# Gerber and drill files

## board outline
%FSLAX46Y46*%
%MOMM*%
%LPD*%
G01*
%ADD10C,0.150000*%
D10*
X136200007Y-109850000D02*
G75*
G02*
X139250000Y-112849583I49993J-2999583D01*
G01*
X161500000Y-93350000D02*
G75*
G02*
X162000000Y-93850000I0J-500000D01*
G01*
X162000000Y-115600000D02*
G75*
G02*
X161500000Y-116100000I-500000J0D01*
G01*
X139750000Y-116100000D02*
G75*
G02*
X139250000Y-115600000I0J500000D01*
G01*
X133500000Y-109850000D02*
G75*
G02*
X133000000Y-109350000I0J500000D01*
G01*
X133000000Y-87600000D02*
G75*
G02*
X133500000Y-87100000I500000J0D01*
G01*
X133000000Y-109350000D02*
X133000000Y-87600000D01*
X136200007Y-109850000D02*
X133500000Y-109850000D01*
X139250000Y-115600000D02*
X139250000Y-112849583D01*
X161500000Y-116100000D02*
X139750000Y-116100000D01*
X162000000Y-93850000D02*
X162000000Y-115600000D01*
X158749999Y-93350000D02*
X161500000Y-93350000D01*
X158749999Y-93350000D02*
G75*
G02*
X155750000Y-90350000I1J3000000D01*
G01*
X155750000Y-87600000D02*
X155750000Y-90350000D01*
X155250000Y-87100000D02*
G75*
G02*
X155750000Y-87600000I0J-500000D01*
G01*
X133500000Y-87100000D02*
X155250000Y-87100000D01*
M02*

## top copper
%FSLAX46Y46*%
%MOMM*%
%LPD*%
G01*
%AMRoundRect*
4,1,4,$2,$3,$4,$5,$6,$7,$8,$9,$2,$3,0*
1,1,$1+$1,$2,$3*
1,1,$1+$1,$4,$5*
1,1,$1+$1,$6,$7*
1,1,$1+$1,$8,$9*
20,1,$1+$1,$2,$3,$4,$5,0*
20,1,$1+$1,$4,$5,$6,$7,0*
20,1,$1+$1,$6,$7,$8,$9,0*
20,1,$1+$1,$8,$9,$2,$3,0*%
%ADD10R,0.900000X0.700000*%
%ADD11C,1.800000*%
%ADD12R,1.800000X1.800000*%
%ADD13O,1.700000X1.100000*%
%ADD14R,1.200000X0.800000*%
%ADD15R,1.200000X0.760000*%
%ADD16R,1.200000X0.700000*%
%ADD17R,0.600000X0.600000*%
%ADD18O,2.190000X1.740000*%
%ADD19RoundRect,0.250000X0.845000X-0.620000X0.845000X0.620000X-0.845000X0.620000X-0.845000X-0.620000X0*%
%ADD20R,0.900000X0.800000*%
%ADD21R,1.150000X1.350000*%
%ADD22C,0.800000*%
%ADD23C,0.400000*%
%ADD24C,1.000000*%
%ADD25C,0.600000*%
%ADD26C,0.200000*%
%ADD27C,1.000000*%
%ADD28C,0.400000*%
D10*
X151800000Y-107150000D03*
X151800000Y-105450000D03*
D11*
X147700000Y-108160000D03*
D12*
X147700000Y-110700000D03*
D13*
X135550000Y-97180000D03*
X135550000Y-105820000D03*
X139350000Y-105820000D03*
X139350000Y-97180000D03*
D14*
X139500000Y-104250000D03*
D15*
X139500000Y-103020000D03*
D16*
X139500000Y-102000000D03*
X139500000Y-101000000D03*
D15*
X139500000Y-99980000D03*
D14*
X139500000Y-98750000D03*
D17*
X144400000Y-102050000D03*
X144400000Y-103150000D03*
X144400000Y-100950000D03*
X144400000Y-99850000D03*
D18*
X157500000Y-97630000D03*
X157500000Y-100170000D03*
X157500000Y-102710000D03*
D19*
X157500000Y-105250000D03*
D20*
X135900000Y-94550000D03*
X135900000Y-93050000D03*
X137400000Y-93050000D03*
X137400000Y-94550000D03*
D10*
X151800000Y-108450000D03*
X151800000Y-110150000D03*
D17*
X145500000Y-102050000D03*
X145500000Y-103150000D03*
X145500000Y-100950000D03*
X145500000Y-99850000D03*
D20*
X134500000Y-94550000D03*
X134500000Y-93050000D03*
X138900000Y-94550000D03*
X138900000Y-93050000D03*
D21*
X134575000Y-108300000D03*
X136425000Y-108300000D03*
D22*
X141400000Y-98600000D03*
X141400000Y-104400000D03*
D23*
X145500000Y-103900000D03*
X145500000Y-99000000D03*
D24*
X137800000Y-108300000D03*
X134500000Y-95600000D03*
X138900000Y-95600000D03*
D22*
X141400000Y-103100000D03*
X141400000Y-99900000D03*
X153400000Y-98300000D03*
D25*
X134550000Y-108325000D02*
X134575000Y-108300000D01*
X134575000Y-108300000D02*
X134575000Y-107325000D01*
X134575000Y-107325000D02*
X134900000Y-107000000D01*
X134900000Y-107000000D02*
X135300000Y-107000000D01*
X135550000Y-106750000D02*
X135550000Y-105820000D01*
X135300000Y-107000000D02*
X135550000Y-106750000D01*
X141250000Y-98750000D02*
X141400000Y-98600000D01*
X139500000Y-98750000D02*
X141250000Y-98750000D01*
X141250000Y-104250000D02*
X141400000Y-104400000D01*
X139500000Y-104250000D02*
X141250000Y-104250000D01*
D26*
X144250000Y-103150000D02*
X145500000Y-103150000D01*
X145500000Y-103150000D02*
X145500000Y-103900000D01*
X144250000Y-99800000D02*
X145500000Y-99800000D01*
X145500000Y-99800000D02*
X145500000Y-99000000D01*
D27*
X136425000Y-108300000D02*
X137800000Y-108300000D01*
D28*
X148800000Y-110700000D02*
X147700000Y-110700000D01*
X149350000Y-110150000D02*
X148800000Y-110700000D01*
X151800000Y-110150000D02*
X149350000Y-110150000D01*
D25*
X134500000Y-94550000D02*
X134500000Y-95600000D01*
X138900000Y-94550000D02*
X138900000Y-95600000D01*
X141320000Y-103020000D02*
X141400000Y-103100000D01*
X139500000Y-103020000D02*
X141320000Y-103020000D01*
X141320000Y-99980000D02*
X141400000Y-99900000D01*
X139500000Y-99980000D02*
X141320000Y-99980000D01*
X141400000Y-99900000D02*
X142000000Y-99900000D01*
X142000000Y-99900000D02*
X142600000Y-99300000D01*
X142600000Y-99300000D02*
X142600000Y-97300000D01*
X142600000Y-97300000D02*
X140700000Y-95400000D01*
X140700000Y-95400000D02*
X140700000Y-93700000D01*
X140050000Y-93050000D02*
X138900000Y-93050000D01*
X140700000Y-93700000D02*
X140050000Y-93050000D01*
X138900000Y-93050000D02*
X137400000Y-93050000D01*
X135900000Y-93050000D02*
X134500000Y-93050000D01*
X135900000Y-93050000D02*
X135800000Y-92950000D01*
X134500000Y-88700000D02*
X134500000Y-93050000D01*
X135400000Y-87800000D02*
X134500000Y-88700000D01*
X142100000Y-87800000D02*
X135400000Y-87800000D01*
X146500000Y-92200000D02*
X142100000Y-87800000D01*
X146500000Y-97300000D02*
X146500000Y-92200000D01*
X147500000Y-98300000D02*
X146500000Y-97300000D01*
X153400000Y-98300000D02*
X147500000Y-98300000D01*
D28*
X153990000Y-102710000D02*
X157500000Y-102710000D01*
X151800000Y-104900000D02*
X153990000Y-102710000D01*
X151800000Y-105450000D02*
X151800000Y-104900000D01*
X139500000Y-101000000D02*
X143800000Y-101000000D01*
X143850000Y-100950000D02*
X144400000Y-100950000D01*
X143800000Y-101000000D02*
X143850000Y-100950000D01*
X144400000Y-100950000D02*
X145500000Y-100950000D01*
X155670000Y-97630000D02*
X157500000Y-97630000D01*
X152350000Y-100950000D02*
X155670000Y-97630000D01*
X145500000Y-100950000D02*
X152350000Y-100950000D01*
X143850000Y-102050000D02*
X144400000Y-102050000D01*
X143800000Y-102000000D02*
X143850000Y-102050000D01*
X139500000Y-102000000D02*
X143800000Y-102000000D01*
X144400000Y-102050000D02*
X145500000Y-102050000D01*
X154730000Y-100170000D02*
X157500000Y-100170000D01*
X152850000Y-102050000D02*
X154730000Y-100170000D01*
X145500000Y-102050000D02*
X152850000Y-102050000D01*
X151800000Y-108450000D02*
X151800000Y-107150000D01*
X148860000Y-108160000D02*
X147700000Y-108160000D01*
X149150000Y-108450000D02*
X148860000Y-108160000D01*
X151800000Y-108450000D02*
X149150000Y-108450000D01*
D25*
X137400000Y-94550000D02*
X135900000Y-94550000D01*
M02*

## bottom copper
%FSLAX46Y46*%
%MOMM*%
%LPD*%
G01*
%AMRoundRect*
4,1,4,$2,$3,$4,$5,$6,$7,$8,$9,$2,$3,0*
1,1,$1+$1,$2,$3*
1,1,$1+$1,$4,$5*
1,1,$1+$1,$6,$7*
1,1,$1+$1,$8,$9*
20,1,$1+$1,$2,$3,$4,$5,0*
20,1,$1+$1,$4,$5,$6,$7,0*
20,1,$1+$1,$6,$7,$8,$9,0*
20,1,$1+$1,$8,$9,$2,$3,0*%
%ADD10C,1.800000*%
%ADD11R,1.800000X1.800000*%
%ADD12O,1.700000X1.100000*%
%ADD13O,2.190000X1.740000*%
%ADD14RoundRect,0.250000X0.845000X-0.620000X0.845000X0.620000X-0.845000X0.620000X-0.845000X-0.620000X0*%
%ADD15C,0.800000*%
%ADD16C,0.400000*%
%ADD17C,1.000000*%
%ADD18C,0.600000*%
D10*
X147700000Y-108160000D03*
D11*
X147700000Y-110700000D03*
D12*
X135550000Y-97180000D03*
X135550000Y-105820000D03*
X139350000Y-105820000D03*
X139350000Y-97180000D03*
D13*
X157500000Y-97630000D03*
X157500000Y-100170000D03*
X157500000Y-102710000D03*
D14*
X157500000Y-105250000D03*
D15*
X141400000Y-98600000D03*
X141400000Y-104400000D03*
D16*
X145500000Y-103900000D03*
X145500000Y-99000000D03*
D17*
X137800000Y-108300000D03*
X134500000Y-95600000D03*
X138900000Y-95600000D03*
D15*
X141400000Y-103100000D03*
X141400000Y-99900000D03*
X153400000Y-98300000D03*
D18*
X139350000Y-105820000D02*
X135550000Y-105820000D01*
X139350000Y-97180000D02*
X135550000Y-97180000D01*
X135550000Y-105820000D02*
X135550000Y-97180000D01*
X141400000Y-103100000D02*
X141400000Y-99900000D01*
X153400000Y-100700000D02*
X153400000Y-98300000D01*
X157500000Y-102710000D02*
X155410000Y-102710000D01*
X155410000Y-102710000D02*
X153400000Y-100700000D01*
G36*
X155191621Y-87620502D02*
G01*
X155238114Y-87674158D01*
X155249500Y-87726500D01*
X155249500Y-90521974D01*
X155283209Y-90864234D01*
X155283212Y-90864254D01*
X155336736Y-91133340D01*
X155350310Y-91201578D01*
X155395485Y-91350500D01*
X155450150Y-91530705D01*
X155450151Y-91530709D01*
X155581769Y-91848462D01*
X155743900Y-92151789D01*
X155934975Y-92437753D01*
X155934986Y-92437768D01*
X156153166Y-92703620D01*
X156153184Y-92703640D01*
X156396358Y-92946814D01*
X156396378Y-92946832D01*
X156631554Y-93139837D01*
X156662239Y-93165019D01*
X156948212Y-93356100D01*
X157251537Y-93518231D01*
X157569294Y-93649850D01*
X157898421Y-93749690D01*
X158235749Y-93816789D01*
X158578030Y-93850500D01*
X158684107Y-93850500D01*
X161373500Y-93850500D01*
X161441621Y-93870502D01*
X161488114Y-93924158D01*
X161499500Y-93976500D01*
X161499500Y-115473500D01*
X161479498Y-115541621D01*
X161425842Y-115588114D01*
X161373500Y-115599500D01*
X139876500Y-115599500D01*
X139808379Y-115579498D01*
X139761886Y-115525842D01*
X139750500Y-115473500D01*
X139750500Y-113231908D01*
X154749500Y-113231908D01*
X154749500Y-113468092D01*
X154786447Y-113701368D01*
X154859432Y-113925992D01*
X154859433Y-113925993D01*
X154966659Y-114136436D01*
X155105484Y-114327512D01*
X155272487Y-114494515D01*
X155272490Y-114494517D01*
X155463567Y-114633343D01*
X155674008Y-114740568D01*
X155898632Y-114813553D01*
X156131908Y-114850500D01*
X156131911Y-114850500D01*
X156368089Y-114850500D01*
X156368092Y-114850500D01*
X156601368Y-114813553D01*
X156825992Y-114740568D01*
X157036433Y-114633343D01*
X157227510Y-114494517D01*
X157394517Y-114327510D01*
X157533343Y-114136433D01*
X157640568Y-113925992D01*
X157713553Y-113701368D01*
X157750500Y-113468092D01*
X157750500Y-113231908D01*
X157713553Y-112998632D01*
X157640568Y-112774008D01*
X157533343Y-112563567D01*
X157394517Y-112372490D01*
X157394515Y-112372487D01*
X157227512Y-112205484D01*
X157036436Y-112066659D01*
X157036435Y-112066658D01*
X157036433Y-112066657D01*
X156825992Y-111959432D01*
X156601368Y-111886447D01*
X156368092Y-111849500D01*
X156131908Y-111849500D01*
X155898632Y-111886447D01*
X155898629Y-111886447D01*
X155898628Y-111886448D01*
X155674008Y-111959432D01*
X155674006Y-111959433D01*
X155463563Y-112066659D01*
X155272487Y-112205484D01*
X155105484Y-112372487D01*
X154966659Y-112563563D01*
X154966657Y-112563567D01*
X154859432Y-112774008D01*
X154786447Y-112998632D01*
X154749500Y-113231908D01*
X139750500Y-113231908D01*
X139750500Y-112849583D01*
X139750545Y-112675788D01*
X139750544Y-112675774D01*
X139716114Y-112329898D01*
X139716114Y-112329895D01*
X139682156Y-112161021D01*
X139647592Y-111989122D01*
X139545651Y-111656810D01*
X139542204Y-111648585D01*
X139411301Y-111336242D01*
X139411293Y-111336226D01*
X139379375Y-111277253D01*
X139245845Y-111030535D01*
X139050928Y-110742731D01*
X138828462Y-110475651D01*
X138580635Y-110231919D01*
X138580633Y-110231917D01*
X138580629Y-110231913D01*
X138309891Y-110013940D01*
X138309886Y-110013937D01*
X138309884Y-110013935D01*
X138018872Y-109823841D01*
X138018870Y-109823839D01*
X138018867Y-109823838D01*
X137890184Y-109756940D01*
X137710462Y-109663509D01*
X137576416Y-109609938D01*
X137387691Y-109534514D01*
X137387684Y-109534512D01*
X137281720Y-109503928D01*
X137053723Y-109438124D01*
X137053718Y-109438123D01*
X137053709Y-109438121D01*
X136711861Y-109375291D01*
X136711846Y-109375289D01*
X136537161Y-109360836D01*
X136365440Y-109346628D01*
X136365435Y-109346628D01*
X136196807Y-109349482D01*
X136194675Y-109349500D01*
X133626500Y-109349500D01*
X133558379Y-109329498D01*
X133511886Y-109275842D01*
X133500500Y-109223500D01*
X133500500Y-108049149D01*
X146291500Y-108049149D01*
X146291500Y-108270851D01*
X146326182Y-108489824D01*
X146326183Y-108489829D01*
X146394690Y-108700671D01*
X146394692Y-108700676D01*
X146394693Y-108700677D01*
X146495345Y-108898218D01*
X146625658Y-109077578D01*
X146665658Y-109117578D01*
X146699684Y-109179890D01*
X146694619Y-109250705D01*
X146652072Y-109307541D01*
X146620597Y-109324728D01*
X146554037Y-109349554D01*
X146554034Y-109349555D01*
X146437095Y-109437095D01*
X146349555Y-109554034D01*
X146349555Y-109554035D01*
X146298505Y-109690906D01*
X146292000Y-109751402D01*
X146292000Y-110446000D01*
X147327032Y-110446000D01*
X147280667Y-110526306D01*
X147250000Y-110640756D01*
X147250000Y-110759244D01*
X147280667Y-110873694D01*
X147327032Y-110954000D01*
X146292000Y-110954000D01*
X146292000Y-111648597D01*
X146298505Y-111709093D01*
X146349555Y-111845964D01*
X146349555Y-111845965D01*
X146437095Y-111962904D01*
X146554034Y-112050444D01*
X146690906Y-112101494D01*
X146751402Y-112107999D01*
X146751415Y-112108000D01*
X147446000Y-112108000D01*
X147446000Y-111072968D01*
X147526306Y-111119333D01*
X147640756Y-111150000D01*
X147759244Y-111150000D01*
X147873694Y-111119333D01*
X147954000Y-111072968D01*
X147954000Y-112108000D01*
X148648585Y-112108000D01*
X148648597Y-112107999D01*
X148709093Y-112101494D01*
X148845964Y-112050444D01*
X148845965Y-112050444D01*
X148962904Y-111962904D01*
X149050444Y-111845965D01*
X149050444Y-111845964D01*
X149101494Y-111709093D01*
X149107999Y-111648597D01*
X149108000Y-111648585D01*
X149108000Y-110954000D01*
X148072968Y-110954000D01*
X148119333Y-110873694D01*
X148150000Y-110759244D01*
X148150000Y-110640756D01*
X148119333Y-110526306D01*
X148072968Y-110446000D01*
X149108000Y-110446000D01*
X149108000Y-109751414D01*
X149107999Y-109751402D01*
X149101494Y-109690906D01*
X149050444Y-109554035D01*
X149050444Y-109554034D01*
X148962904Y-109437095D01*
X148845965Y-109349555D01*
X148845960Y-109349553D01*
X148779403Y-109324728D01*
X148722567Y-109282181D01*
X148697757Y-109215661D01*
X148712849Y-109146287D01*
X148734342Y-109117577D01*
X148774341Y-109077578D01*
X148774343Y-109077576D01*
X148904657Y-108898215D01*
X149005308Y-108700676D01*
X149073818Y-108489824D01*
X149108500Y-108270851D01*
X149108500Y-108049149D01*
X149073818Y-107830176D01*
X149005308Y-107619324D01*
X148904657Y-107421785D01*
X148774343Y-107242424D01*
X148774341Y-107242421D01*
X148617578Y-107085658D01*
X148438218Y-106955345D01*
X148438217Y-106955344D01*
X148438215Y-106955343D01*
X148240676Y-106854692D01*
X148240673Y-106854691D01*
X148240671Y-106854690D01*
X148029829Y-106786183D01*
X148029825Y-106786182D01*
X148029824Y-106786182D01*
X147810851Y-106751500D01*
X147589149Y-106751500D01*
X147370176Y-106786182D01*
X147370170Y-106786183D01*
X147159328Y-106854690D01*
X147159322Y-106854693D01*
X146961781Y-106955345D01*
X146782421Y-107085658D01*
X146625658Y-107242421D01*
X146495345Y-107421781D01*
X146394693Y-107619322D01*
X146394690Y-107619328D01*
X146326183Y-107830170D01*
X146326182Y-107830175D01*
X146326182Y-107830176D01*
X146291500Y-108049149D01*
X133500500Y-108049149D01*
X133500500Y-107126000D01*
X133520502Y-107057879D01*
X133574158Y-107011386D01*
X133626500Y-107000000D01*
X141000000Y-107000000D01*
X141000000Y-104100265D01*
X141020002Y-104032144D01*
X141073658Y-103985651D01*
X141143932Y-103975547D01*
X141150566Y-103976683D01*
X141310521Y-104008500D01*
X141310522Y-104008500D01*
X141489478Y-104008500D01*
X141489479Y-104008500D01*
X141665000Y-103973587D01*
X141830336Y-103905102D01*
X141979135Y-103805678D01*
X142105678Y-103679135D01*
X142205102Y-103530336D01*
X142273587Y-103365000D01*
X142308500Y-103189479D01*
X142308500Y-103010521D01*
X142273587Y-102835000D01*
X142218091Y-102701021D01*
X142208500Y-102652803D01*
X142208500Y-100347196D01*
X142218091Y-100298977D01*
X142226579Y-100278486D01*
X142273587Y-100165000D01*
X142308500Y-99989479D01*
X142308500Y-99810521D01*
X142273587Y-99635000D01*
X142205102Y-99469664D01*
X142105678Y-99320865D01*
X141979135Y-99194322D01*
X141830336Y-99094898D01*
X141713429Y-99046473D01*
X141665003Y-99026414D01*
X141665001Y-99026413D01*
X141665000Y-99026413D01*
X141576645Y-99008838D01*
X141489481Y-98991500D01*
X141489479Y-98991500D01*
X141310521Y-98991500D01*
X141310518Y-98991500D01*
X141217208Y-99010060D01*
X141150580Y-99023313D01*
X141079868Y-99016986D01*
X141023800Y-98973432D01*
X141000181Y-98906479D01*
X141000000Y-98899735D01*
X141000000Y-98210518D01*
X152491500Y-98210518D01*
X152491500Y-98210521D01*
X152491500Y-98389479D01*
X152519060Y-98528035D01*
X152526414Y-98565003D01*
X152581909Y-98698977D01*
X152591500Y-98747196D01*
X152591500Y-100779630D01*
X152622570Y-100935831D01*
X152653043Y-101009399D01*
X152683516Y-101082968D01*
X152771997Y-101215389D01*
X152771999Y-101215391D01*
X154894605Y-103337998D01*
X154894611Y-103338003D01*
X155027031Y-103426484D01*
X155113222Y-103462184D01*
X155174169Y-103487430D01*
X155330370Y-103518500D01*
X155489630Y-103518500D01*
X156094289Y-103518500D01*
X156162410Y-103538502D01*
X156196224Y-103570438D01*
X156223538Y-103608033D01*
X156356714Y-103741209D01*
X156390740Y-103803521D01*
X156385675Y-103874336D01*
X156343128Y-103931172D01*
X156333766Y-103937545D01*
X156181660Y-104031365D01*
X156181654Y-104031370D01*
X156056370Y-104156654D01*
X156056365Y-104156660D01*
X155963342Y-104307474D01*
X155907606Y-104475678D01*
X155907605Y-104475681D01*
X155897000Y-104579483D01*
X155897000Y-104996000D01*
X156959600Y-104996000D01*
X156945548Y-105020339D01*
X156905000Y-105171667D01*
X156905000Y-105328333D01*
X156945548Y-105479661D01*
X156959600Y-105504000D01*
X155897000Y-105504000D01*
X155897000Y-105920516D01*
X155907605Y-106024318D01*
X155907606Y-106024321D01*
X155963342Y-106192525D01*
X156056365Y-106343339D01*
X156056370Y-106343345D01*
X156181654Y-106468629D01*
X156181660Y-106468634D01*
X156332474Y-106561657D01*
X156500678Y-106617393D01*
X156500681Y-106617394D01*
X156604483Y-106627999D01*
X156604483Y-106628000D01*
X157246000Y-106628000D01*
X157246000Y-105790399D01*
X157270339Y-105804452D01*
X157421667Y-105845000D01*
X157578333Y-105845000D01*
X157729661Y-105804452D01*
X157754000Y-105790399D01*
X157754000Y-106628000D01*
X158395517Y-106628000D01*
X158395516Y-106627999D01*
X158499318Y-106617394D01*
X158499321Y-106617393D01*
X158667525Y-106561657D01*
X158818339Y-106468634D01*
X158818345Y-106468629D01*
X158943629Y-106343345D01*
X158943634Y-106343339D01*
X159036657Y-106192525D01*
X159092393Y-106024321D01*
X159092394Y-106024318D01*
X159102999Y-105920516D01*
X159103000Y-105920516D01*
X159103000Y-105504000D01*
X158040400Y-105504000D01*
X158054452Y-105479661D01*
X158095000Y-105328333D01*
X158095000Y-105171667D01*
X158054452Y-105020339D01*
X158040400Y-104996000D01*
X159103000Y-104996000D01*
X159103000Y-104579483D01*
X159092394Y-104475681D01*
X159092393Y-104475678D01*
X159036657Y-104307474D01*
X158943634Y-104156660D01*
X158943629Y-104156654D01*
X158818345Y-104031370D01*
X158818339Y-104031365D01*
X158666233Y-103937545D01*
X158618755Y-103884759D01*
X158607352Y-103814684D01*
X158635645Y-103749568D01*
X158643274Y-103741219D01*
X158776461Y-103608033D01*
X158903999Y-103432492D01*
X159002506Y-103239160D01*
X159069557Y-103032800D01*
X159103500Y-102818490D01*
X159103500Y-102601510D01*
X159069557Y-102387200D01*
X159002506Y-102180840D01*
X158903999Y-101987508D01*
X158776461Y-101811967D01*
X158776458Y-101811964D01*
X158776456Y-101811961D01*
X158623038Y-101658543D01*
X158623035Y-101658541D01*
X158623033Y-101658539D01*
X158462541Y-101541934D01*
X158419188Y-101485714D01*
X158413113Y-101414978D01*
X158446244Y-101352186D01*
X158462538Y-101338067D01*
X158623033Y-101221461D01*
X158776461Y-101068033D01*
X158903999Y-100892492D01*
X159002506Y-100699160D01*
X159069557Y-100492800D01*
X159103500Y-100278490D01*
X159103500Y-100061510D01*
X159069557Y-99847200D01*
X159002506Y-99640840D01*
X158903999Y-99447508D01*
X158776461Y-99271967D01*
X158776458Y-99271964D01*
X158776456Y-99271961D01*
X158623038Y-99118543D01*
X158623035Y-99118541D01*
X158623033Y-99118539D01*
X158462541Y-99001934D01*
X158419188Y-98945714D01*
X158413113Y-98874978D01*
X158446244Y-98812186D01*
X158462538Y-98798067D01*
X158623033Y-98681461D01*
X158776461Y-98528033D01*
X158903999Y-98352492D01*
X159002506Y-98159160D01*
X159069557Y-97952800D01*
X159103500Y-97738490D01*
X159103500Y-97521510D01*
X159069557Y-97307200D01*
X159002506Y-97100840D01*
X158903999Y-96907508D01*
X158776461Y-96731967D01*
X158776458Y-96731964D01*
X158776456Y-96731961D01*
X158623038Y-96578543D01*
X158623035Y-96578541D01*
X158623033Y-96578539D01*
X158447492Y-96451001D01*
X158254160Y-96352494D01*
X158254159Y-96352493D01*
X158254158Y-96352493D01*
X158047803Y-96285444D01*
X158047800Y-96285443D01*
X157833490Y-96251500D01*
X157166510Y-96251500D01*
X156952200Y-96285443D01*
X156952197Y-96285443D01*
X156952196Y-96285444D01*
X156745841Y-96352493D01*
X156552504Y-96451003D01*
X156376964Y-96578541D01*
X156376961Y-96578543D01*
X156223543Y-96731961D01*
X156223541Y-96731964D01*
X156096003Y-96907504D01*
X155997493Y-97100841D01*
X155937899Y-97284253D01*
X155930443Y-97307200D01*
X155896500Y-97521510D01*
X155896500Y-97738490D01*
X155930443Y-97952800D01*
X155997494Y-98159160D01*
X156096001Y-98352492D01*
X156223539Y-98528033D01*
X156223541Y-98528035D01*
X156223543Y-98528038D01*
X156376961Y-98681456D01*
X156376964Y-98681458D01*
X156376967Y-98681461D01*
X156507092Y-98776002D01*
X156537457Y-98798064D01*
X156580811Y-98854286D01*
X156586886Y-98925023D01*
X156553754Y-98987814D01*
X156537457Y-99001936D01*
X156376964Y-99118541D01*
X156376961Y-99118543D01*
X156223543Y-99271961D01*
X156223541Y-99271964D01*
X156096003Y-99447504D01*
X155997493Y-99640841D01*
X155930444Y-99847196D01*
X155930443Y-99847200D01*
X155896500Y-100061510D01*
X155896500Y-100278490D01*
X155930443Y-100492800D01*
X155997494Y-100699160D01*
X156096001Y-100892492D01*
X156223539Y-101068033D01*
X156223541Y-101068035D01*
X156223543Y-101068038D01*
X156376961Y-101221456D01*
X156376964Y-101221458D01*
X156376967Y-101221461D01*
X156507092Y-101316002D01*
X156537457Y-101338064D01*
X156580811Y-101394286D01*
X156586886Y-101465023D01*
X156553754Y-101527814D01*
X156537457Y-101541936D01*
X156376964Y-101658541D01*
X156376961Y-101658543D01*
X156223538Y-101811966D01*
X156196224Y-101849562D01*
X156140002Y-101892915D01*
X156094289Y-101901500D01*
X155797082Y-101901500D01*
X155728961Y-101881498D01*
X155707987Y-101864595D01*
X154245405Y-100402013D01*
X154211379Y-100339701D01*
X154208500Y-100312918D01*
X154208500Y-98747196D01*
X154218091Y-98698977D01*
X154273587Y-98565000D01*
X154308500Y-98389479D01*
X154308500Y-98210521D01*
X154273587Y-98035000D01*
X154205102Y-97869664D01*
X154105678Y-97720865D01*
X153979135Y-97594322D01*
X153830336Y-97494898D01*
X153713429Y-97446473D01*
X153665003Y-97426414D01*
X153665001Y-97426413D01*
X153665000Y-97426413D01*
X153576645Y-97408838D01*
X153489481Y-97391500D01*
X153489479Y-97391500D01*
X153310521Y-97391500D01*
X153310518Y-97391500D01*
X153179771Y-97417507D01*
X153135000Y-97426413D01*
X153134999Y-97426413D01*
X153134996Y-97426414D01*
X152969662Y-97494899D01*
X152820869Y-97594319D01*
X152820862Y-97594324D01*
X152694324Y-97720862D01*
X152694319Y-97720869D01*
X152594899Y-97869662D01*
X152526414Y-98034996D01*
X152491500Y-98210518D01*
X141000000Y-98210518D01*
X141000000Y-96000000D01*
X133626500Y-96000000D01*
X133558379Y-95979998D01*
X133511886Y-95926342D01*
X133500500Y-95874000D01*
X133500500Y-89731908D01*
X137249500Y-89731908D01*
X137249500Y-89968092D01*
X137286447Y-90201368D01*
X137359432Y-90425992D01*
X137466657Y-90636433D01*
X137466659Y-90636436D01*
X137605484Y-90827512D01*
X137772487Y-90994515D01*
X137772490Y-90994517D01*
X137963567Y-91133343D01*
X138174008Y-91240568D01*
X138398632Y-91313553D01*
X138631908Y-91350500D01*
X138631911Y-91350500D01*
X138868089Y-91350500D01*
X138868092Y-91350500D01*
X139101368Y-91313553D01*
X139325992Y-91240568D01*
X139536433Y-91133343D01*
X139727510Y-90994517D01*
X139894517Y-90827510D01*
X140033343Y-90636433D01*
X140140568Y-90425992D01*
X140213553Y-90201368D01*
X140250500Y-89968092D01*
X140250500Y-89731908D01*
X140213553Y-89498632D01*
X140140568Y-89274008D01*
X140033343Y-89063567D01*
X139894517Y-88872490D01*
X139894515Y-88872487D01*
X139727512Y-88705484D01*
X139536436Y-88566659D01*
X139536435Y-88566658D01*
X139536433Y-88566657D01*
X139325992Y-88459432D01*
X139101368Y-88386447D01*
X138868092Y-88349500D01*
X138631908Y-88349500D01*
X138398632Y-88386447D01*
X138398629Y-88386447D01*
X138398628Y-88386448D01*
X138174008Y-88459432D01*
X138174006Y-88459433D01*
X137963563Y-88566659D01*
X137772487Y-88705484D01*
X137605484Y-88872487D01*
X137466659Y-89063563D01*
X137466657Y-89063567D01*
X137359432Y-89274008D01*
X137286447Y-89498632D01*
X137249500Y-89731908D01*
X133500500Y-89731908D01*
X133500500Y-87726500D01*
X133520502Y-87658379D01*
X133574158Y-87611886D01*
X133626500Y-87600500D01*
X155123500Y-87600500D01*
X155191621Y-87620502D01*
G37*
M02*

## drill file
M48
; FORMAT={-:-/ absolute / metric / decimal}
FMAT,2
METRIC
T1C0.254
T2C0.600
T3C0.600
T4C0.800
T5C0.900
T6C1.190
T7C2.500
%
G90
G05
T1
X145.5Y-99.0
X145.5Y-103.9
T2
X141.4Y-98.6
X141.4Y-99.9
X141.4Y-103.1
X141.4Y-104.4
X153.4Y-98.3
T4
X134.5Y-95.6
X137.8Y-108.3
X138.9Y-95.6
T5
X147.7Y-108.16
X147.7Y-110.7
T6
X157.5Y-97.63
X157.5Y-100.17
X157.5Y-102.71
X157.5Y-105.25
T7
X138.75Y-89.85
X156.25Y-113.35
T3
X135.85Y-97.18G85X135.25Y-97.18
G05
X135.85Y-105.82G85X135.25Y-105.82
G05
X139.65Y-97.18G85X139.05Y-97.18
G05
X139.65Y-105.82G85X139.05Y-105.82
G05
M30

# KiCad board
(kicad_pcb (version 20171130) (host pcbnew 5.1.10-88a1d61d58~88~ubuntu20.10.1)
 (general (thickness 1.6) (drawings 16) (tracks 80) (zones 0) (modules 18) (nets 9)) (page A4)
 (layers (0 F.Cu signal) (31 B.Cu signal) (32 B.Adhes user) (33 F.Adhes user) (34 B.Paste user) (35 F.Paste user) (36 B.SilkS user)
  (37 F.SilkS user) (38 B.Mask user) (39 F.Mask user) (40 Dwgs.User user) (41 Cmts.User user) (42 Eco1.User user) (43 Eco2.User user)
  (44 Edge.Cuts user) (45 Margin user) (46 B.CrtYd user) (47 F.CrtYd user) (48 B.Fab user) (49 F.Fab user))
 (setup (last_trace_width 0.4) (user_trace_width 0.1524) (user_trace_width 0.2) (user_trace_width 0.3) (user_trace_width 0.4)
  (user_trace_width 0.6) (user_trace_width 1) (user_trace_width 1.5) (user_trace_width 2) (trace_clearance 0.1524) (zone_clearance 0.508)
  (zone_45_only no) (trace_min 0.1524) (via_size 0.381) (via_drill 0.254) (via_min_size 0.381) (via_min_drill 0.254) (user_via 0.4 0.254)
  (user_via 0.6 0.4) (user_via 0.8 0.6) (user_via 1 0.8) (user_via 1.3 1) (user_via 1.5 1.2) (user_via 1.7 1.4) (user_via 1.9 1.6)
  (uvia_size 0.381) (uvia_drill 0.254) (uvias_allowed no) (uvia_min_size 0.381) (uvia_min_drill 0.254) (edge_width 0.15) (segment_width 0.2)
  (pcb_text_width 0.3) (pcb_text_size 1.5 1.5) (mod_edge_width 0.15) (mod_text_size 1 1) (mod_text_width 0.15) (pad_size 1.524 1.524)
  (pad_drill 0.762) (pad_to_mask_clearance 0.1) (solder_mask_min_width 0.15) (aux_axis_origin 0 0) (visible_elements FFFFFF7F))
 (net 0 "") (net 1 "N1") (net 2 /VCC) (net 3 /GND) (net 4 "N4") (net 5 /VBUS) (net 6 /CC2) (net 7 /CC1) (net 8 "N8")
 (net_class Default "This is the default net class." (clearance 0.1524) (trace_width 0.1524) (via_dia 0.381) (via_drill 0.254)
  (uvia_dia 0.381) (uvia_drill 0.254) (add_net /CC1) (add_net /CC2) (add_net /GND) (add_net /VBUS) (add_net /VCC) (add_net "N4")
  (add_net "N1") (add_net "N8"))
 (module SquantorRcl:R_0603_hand (layer F.Cu) (at 151.8 106.3 270)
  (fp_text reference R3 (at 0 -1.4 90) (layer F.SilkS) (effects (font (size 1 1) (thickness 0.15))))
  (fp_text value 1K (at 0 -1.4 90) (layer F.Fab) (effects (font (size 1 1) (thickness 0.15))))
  (pad 2 smd rect (at 0.85 0 270) (size 0.7 0.9) (layers F.Cu F.Paste F.Mask) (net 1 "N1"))
  (pad 1 smd rect (at -0.85 0 270) (size 0.7 0.9) (layers F.Cu F.Paste F.Mask) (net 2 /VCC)))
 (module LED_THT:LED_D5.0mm (layer F.Cu) (at 147.7 110.7 90)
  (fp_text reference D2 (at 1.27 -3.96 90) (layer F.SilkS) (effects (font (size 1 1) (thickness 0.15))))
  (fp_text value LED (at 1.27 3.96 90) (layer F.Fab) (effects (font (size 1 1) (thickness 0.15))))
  (pad 2 thru_hole circle (at 2.54 0 90) (size 1.8 1.8) (drill 0.9) (layers *.Cu *.Mask) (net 1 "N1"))
  (pad 1 thru_hole rect (at 0 0 90) (size 1.8 1.8) (drill 0.9) (layers *.Cu *.Mask) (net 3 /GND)))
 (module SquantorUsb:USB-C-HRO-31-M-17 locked (layer F.Cu) (at 139.5 101.5 270)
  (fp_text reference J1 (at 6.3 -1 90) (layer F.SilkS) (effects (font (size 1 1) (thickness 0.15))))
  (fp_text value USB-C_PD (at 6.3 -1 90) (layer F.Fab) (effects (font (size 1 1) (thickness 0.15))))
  (pad S thru_hole oval (at -4.32 3.95 270) (size 1.1 1.7) (drill oval 0.6 1.2) (layers *.Cu *.Mask) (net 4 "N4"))
  (pad S thru_hole oval (at 4.32 3.95 270) (size 1.1 1.7) (drill oval 0.6 1.2) (layers *.Cu *.Mask) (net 4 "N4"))
  (pad S thru_hole oval (at 4.32 0.15 270) (size 1.1 1.7) (drill oval 0.6 1.2) (layers *.Cu *.Mask) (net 4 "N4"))
  (pad S thru_hole oval (at -4.32 0.15 270) (size 1.1 1.7) (drill oval 0.6 1.2) (layers *.Cu *.Mask) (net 4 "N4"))
  (pad A12 smd rect (at 2.75 0 270) (size 0.8 1.2) (layers F.Cu F.Paste F.Mask) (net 3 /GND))
  (pad A9 smd rect (at 1.52 0 270) (size 0.76 1.2) (layers F.Cu F.Paste F.Mask) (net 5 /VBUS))
  (pad B5 smd rect (at 0.5 0 270) (size 0.7 1.2) (layers F.Cu F.Paste F.Mask) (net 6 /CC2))
  (pad A5 smd rect (at -0.5 0 270) (size 0.7 1.2) (layers F.Cu F.Paste F.Mask) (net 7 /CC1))
  (pad B9 smd rect (at -1.52 0 270) (size 0.76 1.2) (layers F.Cu F.Paste F.Mask) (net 5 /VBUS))
  (pad B12 smd rect (at -2.75 0 270) (size 0.8 1.2) (layers F.Cu F.Paste F.Mask) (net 3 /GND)))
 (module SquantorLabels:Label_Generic (layer B.Cu) (at 148.5 104.75 180)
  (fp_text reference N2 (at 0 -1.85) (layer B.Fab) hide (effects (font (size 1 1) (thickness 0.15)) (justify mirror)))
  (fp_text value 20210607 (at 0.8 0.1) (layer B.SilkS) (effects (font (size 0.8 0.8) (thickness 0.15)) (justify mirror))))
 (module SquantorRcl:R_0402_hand (layer F.Cu) (at 144.4 102.6 90)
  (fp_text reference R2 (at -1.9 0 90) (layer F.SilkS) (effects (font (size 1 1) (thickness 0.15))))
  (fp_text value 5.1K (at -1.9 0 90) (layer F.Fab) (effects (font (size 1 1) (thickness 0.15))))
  (pad 2 smd rect (at 0.55 0 90) (size 0.6 0.6) (layers F.Cu F.Paste F.Mask) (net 6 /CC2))
  (pad 1 smd rect (at -0.55 0 90) (size 0.6 0.6) (layers F.Cu F.Paste F.Mask) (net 3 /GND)))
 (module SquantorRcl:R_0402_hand (layer F.Cu) (at 144.4 100.4 270)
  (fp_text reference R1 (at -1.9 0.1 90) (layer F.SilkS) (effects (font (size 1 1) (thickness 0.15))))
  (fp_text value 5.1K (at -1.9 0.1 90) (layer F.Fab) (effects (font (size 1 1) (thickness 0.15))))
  (pad 2 smd rect (at 0.55 0 270) (size 0.6 0.6) (layers F.Cu F.Paste F.Mask) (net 7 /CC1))
  (pad 1 smd rect (at -0.55 0 270) (size 0.6 0.6) (layers F.Cu F.Paste F.Mask) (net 3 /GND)))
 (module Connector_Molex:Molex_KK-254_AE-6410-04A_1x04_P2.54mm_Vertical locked (layer F.Cu) (at 157.5 105.25 90)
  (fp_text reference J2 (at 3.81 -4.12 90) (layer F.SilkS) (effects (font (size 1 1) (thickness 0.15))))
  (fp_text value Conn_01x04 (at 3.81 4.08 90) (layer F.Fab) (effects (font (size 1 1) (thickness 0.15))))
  (pad 4 thru_hole oval (at 7.62 0 90) (size 1.74 2.19) (drill 1.19) (layers *.Cu *.Mask) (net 7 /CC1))
  (pad 3 thru_hole oval (at 5.08 0 90) (size 1.74 2.19) (drill 1.19) (layers *.Cu *.Mask) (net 6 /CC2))
  (pad 2 thru_hole oval (at 2.54 0 90) (size 1.74 2.19) (drill 1.19) (layers *.Cu *.Mask) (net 2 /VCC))
  (pad 1 thru_hole roundrect (at 0 0 90) (size 1.74 2.19) (drill 1.19) (layers *.Cu *.Mask) (roundrect_rratio 0.143678) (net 3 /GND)))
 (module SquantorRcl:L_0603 (layer F.Cu) (at 135.9 93.8 270)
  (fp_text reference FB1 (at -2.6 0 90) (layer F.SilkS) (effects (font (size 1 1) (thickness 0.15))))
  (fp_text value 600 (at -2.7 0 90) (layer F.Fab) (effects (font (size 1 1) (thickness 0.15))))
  (pad 2 smd rect (at 0.75 0 270) (size 0.8 0.9) (layers F.Cu F.Paste F.Mask) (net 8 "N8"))
  (pad 1 smd rect (at -0.75 0 270) (size 0.8 0.9) (layers F.Cu F.Paste F.Mask) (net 2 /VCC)))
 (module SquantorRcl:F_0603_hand (layer F.Cu) (at 137.4 93.8 90)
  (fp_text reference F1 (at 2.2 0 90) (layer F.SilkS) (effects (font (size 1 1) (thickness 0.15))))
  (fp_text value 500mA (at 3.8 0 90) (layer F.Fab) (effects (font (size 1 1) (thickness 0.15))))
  (pad 2 smd rect (at 0.75 0 90) (size 0.8 0.9) (layers F.Cu F.Paste F.Mask) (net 5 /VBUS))
  (pad 1 smd rect (at -0.75 0 90) (size 0.8 0.9) (layers F.Cu F.Paste F.Mask) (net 8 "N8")))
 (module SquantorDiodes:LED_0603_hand (layer F.Cu) (at 151.8 109.3 90)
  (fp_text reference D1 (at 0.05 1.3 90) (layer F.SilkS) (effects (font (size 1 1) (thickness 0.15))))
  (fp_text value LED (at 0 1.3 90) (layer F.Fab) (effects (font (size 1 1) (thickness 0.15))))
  (pad 2 smd rect (at 0.85 0 90) (size 0.7 0.9) (layers F.Cu F.Paste F.Mask) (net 1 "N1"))
  (pad 1 smd rect (at -0.85 0 90) (size 0.7 0.9) (layers F.Cu F.Paste F.Mask) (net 3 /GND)))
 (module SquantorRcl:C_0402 (layer F.Cu) (at 145.5 102.6 90)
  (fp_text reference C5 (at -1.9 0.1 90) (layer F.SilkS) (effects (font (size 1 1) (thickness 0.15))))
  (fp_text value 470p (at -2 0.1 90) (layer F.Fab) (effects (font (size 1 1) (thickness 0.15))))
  (pad 2 smd rect (at 0.55 0 90) (size 0.6 0.6) (layers F.Cu F.Paste F.Mask) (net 6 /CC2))
  (pad 1 smd rect (at -0.55 0 90) (size 0.6 0.6) (layers F.Cu F.Paste F.Mask) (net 3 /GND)))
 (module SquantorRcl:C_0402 (layer F.Cu) (at 145.5 100.4 270)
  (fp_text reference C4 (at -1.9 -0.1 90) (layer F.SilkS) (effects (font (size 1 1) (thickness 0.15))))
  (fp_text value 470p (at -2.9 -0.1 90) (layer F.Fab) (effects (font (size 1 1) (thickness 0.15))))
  (pad 2 smd rect (at 0.55 0 270) (size 0.6 0.6) (layers F.Cu F.Paste F.Mask) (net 7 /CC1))
  (pad 1 smd rect (at -0.55 0 270) (size 0.6 0.6) (layers F.Cu F.Paste F.Mask) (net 3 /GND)))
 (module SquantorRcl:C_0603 (layer F.Cu) (at 134.5 93.8 270)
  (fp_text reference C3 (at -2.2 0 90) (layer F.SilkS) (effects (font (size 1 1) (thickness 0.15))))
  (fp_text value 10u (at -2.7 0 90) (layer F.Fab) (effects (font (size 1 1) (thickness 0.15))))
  (pad 2 smd rect (at 0.75 0 270) (size 0.8 0.9) (layers F.Cu F.Paste F.Mask) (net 3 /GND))
  (pad 1 smd rect (at -0.75 0 270) (size 0.8 0.9) (layers F.Cu F.Paste F.Mask) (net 2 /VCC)))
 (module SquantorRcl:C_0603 (layer F.Cu) (at 138.9 93.8 270)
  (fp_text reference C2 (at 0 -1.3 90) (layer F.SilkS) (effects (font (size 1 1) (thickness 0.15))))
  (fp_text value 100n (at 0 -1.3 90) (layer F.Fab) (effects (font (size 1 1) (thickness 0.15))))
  (pad 2 smd rect (at 0.75 0 270) (size 0.8 0.9) (layers F.Cu F.Paste F.Mask) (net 3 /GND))
  (pad 1 smd rect (at -0.75 0 270) (size 0.8 0.9) (layers F.Cu F.Paste F.Mask) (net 5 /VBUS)))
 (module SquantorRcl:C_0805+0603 (layer F.Cu) (at 135.5 108.3)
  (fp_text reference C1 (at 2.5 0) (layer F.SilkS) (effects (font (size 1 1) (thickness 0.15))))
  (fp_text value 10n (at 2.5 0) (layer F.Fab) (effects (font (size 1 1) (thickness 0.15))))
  (pad 1 smd rect (at -0.925 0) (size 1.15 1.35) (layers F.Cu F.Paste F.Mask) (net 4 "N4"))
  (pad 2 smd rect (at 0.925 0) (size 1.15 1.35) (layers F.Cu F.Paste F.Mask) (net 3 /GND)))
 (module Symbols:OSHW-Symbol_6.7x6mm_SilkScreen (layer B.Cu) (at 148 101 180)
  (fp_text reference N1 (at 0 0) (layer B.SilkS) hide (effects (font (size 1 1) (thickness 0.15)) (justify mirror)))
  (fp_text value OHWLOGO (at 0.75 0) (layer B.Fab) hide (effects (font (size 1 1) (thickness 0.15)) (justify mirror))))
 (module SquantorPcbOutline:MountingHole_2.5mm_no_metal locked (layer F.Cu) (at 138.75 89.85)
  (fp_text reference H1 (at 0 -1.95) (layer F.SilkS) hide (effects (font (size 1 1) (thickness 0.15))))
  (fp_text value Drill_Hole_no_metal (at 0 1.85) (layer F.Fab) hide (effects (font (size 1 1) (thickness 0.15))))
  (pad "" np_thru_hole circle (at 0 0) (size 2.5 2.5) (drill 2.5) (layers *.Cu *.Mask)))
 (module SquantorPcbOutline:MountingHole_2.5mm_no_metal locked (layer F.Cu) (at 156.25 113.35)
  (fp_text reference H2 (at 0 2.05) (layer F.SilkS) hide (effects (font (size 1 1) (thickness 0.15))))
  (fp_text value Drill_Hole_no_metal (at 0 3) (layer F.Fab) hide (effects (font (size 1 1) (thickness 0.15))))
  (pad "" np_thru_hole circle (at 0 0) (size 2.5 2.5) (drill 2.5) (layers *.Cu *.Mask)))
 (gr_arc (start 136.25 112.849583) (end 139.25 112.849583) (angle -90.95484125) (layer Edge.Cuts) (width 0.15))
 (gr_arc (start 161.5 93.85) (end 162 93.85) (angle -90) (layer Edge.Cuts) (width 0.15))
 (gr_arc (start 161.5 115.6) (end 161.5 116.1) (angle -90) (layer Edge.Cuts) (width 0.15))
 (gr_arc (start 139.75 115.6) (end 139.25 115.6) (angle -90) (layer Edge.Cuts) (width 0.15))
 (gr_arc (start 133.5 109.35) (end 133 109.35) (angle -90) (layer Edge.Cuts) (width 0.15))
 (gr_arc (start 133.5 87.6) (end 133.5 87.1) (angle -90) (layer Edge.Cuts) (width 0.15))
 (gr_line (start 133 109.35) (end 133 87.6) (layer Edge.Cuts) (width 0.15))
 (gr_line (start 136.200007 109.85) (end 133.5 109.85) (layer Edge.Cuts) (width 0.15))
 (gr_line (start 139.25 115.6) (end 139.25 112.849583) (layer Edge.Cuts) (width 0.15))
 (gr_line (start 161.5 116.1) (end 139.75 116.1) (layer Edge.Cuts) (width 0.15))
 (gr_line (start 162 93.85) (end 162 115.6) (layer Edge.Cuts) (width 0.15))
 (gr_line (start 158.749999 93.35) (end 161.5 93.35) (layer Edge.Cuts) (width 0.15))
 (gr_arc (start 158.75 90.35) (end 155.75 90.35) (angle -89.9999809) (layer Edge.Cuts) (width 0.15))
 (gr_line (start 155.75 87.6) (end 155.75 90.35) (layer Edge.Cuts) (width 0.15))
 (gr_arc (start 155.25 87.6) (end 155.75 87.6) (angle -90) (layer Edge.Cuts) (width 0.15))
 (gr_line (start 133.5 87.1) (end 155.25 87.1) (layer Edge.Cuts) (width 0.15))
 (segment (start 139.35 105.82) (end 135.55 105.82) (width 0.6) (layer B.Cu) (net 4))
 (segment (start 139.35 97.18) (end 135.55 97.18) (width 0.6) (layer B.Cu) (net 4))
 (segment (start 135.55 105.82) (end 135.55 97.18) (width 0.6) (layer B.Cu) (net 4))
 (segment (start 134.55 108.325) (end 134.575 108.3) (width 0.6) (layer F.Cu) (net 4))
 (segment (start 134.575 108.3) (end 134.575 107.325) (width 0.6) (layer F.Cu) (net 4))
 (segment (start 134.575 107.325) (end 134.9 107) (width 0.6) (layer F.Cu) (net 4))
 (segment (start 134.9 107) (end 135.3 107) (width 0.6) (layer F.Cu) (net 4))
 (segment (start 135.55 106.75) (end 135.55 105.82) (width 0.6) (layer F.Cu) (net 4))
 (segment (start 135.3 107) (end 135.55 106.75) (width 0.6) (layer F.Cu) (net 4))
 (via (at 141.4 98.6) (size 0.8) (drill 0.6) (layers F.Cu B.Cu) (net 3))
 (segment (start 141.25 98.75) (end 141.4 98.6) (width 0.6) (layer F.Cu) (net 3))
 (segment (start 139.5 98.75) (end 141.25 98.75) (width 0.6) (layer F.Cu) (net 3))
 (via (at 141.4 104.4) (size 0.8) (drill 0.6) (layers F.Cu B.Cu) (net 3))
 (segment (start 141.25 104.25) (end 141.4 104.4) (width 0.6) (layer F.Cu) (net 3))
 (segment (start 139.5 104.25) (end 141.25 104.25) (width 0.6) (layer F.Cu) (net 3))
 (segment (start 144.25 103.15) (end 145.5 103.15) (width 0.2) (layer F.Cu) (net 3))
 (via (at 145.5 103.9) (size 0.4) (drill 0.254) (layers F.Cu B.Cu) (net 3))
 (segment (start 145.5 103.15) (end 145.5 103.9) (width 0.2) (layer F.Cu) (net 3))
 (segment (start 144.25 99.8) (end 145.5 99.8) (width 0.2) (layer F.Cu) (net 3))
 (via (at 145.5 99) (size 0.4) (drill 0.254) (layers F.Cu B.Cu) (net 3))
 (segment (start 145.5 99.8) (end 145.5 99) (width 0.2) (layer F.Cu) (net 3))
 (via (at 137.8 108.3) (size 1) (drill 0.8) (layers F.Cu B.Cu) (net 3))
 (segment (start 136.425 108.3) (end 137.8 108.3) (width 1) (layer F.Cu) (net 3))
 (segment (start 148.8 110.7) (end 147.7 110.7) (width 0.4) (layer F.Cu) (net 3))
 (segment (start 149.35 110.15) (end 148.8 110.7) (width 0.4) (layer F.Cu) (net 3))
 (segment (start 151.8 110.15) (end 149.35 110.15) (width 0.4) (layer F.Cu) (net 3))
 (segment (start 134.5 94.55) (end 134.5 95.6) (width 0.6) (layer F.Cu) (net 3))
 (via (at 134.5 95.6) (size 1) (drill 0.8) (layers F.Cu B.Cu) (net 3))
 (segment (start 138.9 94.55) (end 138.9 95.6) (width 0.6) (layer F.Cu) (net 3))
 (via (at 138.9 95.6) (size 1) (drill 0.8) (layers F.Cu B.Cu) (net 3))
 (via (at 141.4 103.1) (size 0.8) (drill 0.6) (layers F.Cu B.Cu) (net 5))
 (segment (start 141.32 103.02) (end 141.4 103.1) (width 0.6) (layer F.Cu) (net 5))
 (segment (start 139.5 103.02) (end 141.32 103.02) (width 0.6) (layer F.Cu) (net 5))
 (via (at 141.4 99.9) (size 0.8) (drill 0.6) (layers F.Cu B.Cu) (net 5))
 (segment (start 141.32 99.98) (end 141.4 99.9) (width 0.6) (layer F.Cu) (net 5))
 (segment (start 139.5 99.98) (end 141.32 99.98) (width 0.6) (layer F.Cu) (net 5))
 (segment (start 141.4 103.1) (end 141.4 99.9) (width 0.6) (layer B.Cu) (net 5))
 (segment (start 141.4 99.9) (end 142 99.9) (width 0.6) (layer F.Cu) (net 5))
 (segment (start 142 99.9) (end 142.6 99.3) (width 0.6) (layer F.Cu) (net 5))
 (segment (start 142.6 99.3) (end 142.6 97.3) (width 0.6) (layer F.Cu) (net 5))
 (segment (start 142.6 97.3) (end 140.7 95.4) (width 0.6) (layer F.Cu) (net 5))
 (segment (start 140.7 95.4) (end 140.7 93.7) (width 0.6) (layer F.Cu) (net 5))
 (segment (start 140.05 93.05) (end 138.9 93.05) (width 0.6) (layer F.Cu) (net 5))
 (segment (start 140.7 93.7) (end 140.05 93.05) (width 0.6) (layer F.Cu) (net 5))
 (segment (start 138.9 93.05) (end 137.4 93.05) (width 0.6) (layer F.Cu) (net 5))
 (segment (start 135.9 93.05) (end 134.5 93.05) (width 0.6) (layer F.Cu) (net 2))
 (segment (start 153.4 100.7) (end 153.4 98.3) (width 0.6) (layer B.Cu) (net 2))
 (via (at 153.4 98.3) (size 0.8) (drill 0.6) (layers F.Cu B.Cu) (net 2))
 (segment (start 157.5 102.71) (end 155.41 102.71) (width 0.6) (layer B.Cu) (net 2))
 (segment (start 155.41 102.71) (end 153.4 100.7) (width 0.6) (layer B.Cu) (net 2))
 (segment (start 135.9 93.05) (end 135.8 92.95) (width 0.6) (layer F.Cu) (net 2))
 (segment (start 134.5 88.7) (end 134.5 93.05) (width 0.6) (layer F.Cu) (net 2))
 (segment (start 135.4 87.8) (end 134.5 88.7) (width 0.6) (layer F.Cu) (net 2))
 (segment (start 142.1 87.8) (end 135.4 87.8) (width 0.6) (layer F.Cu) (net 2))
 (segment (start 146.5 92.2) (end 142.1 87.8) (width 0.6) (layer F.Cu) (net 2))
 (segment (start 146.5 97.3) (end 146.5 92.2) (width 0.6) (layer F.Cu) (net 2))
 (segment (start 147.5 98.3) (end 146.5 97.3) (width 0.6) (layer F.Cu) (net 2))
 (segment (start 153.4 98.3) (end 147.5 98.3) (width 0.6) (layer F.Cu) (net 2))
 (segment (start 153.99 102.71) (end 157.5 102.71) (width 0.4) (layer F.Cu) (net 2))
 (segment (start 151.8 104.9) (end 153.99 102.71) (width 0.4) (layer F.Cu) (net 2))
 (segment (start 151.8 105.45) (end 151.8 104.9) (width 0.4) (layer F.Cu) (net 2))
 (segment (start 139.5 101) (end 143.8 101) (width 0.4) (layer F.Cu) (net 7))
 (segment (start 143.85 100.95) (end 144.4 100.95) (width 0.4) (layer F.Cu) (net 7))
 (segment (start 143.8 101) (end 143.85 100.95) (width 0.4) (layer F.Cu) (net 7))
 (segment (start 144.4 100.95) (end 145.5 100.95) (width 0.4) (layer F.Cu) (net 7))
 (segment (start 155.67 97.63) (end 157.5 97.63) (width 0.4) (layer F.Cu) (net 7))
 (segment (start 152.35 100.95) (end 155.67 97.63) (width 0.4) (layer F.Cu) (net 7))
 (segment (start 145.5 100.95) (end 152.35 100.95) (width 0.4) (layer F.Cu) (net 7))
 (segment (start 143.85 102.05) (end 144.4 102.05) (width 0.4) (layer F.Cu) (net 6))
 (segment (start 143.8 102) (end 143.85 102.05) (width 0.4) (layer F.Cu) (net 6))
 (segment (start 139.5 102) (end 143.8 102) (width 0.4) (layer F.Cu) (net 6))
 (segment (start 144.4 102.05) (end 145.5 102.05) (width 0.4) (layer F.Cu) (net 6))
 (segment (start 154.73 100.17) (end 157.5 100.17) (width 0.4) (layer F.Cu) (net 6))
 (segment (start 152.85 102.05) (end 154.73 100.17) (width 0.4) (layer F.Cu) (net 6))
 (segment (start 145.5 102.05) (end 152.85 102.05) (width 0.4) (layer F.Cu) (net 6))
 (segment (start 151.8 108.45) (end 151.8 107.15) (width 0.4) (layer F.Cu) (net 1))
 (segment (start 148.86 108.16) (end 147.7 108.16) (width 0.4) (layer F.Cu) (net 1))
 (segment (start 149.15 108.45) (end 148.86 108.16) (width 0.4) (layer F.Cu) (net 1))
 (segment (start 151.8 108.45) (end 149.15 108.45) (width 0.4) (layer F.Cu) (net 1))
 (segment (start 137.4 94.55) (end 135.9 94.55) (width 0.6) (layer F.Cu) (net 8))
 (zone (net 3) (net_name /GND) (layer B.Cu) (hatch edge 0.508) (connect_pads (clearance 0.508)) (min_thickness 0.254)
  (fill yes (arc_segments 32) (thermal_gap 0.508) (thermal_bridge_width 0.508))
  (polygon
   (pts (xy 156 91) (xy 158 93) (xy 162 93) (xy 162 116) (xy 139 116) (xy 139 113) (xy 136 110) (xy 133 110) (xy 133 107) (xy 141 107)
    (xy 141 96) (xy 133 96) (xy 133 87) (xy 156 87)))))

